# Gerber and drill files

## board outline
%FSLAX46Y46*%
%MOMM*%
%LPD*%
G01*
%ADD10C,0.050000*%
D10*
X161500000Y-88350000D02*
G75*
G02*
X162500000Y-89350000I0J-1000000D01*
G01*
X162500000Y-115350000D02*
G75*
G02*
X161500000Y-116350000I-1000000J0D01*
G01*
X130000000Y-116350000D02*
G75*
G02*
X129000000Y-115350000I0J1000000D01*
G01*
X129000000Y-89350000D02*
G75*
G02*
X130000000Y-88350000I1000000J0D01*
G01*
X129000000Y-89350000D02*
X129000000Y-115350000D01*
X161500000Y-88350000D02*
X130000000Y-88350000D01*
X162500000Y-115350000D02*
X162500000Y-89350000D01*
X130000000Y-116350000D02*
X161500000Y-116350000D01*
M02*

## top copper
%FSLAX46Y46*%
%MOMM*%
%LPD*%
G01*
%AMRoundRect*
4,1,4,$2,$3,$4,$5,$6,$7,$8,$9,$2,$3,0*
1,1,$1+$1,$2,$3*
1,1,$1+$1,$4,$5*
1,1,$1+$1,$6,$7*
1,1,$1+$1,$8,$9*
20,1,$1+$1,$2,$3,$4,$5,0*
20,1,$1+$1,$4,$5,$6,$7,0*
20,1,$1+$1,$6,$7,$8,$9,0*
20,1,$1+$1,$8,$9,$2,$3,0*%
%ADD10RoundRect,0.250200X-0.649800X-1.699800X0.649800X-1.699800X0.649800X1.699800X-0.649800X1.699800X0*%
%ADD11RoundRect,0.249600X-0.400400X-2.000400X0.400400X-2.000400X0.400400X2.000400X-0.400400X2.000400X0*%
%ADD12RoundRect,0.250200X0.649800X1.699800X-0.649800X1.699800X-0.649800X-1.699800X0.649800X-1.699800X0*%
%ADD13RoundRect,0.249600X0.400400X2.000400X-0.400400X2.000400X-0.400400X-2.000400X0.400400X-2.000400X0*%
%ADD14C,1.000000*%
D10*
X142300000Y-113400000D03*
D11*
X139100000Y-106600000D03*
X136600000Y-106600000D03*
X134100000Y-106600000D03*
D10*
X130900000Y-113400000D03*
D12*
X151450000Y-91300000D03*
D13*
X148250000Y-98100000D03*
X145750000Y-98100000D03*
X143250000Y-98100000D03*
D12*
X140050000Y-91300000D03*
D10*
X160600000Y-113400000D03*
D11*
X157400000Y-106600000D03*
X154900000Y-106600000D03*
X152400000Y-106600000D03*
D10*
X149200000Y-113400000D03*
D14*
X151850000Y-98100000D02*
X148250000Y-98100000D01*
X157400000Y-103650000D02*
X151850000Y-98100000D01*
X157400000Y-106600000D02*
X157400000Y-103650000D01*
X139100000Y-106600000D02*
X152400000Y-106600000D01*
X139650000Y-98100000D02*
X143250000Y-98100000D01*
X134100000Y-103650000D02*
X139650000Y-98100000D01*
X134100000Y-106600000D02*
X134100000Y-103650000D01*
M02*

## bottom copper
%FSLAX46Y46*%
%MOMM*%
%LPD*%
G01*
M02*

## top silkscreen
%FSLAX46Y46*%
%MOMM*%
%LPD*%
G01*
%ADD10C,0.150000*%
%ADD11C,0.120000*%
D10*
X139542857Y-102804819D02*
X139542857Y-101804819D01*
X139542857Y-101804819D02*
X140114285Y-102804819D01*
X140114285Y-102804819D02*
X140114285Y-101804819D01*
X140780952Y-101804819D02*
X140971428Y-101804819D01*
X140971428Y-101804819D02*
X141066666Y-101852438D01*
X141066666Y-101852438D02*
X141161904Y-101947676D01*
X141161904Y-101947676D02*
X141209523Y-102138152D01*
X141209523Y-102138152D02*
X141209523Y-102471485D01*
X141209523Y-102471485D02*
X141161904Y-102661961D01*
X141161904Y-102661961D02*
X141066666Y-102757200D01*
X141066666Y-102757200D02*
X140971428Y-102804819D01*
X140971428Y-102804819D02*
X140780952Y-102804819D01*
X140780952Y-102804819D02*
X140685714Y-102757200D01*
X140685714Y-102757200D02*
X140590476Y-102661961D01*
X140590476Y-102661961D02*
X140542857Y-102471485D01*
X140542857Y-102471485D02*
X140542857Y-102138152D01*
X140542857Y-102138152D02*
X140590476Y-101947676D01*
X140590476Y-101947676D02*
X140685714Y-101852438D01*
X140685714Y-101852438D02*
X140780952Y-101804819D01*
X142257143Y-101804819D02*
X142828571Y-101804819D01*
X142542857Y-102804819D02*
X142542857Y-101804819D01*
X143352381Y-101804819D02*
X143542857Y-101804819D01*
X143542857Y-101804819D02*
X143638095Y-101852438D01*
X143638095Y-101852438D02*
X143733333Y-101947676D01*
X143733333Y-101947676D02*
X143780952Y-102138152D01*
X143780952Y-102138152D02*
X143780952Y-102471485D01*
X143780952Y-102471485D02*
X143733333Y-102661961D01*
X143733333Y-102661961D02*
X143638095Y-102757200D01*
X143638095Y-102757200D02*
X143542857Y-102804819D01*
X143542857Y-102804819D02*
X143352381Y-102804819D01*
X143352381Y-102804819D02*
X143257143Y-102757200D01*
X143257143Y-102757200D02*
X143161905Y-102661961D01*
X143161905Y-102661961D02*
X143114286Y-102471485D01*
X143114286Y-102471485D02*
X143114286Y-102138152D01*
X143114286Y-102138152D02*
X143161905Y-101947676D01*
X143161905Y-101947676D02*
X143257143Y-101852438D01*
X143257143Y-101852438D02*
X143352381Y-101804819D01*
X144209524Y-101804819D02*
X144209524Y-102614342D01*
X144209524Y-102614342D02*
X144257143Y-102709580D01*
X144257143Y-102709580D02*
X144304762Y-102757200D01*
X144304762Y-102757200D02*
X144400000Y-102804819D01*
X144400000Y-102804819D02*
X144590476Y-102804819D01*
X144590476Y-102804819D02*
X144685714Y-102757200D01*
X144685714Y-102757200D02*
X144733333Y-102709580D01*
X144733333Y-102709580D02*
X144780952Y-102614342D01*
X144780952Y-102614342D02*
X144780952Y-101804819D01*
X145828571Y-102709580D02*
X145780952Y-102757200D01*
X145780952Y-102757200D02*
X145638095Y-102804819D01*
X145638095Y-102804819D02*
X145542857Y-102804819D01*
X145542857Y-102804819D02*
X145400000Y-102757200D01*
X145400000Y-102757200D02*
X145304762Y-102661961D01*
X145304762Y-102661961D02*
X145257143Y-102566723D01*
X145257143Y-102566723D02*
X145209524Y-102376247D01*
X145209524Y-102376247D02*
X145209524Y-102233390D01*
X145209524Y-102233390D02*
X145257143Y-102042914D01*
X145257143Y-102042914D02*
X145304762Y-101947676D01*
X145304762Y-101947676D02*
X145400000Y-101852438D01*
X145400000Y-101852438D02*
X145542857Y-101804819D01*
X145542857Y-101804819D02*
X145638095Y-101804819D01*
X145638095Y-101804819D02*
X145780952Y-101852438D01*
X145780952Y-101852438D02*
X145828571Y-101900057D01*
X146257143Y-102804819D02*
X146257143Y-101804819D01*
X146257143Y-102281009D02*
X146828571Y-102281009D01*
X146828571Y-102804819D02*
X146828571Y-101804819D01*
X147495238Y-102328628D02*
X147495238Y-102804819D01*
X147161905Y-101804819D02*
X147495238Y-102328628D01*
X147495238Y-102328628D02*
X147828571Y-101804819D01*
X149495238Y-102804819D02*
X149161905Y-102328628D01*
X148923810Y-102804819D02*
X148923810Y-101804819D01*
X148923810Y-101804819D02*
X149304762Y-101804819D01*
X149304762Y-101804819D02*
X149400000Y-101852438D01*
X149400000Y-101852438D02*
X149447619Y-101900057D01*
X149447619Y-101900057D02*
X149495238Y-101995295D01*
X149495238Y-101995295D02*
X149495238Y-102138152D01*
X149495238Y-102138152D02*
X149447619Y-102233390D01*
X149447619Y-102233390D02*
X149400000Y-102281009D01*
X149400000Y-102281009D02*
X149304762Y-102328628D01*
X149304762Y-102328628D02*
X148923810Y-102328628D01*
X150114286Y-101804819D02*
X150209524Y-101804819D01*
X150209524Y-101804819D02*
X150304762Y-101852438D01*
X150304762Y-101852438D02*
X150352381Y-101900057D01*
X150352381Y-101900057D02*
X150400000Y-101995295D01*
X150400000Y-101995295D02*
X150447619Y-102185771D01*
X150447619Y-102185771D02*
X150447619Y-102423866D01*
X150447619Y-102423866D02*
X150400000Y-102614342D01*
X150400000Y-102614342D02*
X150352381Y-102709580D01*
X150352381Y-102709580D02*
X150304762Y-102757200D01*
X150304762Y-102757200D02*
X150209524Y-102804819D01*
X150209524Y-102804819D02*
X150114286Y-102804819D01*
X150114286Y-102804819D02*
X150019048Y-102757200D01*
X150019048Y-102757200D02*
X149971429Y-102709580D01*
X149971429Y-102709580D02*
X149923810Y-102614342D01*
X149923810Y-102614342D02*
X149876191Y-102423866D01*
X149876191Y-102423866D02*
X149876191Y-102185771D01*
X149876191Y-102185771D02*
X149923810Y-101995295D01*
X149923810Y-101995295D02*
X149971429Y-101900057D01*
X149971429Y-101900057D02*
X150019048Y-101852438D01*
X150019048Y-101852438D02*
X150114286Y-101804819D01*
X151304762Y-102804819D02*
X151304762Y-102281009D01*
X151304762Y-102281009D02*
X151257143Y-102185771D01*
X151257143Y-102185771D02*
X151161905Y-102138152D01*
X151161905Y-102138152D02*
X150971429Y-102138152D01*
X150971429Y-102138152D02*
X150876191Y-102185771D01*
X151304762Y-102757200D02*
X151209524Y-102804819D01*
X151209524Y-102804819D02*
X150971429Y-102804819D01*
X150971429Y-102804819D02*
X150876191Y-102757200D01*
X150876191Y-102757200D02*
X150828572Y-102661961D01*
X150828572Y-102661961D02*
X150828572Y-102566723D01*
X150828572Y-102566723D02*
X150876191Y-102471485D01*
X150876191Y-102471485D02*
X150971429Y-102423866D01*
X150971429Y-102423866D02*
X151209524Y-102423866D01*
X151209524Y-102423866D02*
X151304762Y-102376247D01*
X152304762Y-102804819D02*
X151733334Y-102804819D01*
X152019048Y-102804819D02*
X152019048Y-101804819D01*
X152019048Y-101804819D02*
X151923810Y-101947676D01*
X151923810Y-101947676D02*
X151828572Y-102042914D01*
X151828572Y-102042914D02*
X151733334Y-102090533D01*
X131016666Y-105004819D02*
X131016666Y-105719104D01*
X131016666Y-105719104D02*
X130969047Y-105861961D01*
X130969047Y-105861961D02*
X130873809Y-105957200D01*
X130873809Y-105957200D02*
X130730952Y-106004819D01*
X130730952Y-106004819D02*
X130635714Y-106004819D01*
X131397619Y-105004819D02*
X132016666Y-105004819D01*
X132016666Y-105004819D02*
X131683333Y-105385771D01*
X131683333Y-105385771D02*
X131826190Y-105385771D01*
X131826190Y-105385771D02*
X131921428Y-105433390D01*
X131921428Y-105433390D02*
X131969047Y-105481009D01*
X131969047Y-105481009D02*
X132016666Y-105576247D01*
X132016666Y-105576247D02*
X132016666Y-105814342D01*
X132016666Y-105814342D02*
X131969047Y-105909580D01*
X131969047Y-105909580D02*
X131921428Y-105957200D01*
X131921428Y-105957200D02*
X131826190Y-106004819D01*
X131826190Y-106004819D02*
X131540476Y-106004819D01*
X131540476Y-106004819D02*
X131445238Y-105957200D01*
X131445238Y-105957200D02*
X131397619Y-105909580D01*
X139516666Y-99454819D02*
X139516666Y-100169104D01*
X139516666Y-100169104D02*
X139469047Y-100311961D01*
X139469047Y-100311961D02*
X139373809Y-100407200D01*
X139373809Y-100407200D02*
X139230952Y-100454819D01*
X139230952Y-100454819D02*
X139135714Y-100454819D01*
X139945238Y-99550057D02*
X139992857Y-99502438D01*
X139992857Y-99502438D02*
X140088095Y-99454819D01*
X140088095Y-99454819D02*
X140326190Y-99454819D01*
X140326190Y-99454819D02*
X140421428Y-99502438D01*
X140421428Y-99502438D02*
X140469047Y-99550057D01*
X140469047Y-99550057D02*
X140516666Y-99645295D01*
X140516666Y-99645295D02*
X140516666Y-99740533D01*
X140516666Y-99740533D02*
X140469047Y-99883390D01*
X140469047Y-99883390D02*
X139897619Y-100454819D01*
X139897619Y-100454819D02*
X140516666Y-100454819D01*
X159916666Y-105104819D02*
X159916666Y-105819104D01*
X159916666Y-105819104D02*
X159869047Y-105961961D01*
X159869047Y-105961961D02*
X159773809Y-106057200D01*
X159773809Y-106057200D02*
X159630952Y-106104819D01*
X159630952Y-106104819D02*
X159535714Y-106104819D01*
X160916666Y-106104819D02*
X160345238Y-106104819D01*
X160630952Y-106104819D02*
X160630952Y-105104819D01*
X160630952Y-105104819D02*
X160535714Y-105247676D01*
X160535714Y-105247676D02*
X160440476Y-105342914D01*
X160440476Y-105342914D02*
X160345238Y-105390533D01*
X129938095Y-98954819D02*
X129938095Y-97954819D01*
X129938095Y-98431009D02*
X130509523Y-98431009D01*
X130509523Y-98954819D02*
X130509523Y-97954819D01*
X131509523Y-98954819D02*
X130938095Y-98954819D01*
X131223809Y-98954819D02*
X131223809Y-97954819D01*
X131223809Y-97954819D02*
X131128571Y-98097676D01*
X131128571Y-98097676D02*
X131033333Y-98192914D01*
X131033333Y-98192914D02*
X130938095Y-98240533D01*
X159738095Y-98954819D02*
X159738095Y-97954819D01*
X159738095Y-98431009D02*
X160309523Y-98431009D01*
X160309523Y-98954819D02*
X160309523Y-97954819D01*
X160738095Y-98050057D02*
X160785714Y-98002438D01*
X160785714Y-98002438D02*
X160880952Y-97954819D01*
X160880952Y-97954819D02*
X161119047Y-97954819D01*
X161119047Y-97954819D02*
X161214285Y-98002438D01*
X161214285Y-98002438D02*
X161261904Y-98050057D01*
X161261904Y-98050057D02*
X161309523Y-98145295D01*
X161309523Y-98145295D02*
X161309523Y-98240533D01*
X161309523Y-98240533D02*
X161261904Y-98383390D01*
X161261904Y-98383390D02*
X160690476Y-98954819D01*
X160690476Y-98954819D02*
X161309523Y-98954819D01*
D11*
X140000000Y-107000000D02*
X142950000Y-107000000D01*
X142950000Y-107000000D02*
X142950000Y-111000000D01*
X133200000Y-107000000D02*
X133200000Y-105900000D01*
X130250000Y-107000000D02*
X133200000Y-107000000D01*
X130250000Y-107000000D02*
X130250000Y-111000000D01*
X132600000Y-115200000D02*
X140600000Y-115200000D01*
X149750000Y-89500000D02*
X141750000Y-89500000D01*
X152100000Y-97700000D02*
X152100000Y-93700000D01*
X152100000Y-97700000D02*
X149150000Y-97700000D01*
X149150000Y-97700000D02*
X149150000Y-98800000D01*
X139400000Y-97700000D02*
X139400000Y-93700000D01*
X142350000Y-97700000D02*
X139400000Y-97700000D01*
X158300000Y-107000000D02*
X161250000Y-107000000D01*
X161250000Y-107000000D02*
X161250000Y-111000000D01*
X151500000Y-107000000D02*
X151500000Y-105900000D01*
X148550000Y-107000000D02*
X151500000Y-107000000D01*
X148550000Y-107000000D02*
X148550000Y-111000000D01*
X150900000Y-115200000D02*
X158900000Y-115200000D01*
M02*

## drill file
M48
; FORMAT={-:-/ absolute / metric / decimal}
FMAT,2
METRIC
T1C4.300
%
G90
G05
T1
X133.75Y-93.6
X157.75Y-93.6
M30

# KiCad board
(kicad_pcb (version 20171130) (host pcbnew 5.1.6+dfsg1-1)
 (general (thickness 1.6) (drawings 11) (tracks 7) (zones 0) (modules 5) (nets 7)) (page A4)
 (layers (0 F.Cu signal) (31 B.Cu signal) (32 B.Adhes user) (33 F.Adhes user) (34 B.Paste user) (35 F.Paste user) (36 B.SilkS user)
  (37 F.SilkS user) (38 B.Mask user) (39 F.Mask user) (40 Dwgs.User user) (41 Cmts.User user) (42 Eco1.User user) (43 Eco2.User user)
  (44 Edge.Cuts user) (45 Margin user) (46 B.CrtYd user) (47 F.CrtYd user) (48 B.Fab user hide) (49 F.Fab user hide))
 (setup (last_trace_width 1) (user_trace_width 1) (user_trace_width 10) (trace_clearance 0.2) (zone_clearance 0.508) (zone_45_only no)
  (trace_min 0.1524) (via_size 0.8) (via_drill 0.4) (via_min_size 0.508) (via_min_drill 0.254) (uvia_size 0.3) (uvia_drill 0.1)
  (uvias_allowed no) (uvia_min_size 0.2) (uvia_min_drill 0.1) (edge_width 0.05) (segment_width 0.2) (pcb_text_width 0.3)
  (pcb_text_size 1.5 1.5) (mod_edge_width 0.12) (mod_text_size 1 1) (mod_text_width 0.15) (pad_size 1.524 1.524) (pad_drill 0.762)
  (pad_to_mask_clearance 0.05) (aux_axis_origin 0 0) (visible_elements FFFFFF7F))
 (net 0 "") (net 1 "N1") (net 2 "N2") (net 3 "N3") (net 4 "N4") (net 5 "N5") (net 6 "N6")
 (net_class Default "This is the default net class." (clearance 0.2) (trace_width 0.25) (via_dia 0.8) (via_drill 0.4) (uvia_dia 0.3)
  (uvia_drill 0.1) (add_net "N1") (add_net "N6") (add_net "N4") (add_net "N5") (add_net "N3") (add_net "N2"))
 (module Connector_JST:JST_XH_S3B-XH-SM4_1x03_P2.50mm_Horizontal (layer F.Cu) (at 136.6 111.1)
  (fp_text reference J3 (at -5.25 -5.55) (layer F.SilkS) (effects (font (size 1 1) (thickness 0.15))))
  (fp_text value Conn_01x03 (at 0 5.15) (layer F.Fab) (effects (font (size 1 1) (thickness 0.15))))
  (fp_line (start 3.4 -4.1) (end 6.35 -4.1) (layer F.SilkS) (width 0.12))
  (fp_line (start 6.35 -4.1) (end 6.35 -0.1) (layer F.SilkS) (width 0.12))
  (fp_line (start -3.4 -4.1) (end -3.4 -5.2) (layer F.SilkS) (width 0.12))
  (fp_line (start -6.35 -4.1) (end -3.4 -4.1) (layer F.SilkS) (width 0.12))
  (fp_line (start -6.35 -4.1) (end -6.35 -0.1) (layer F.SilkS) (width 0.12))
  (fp_line (start -4 4.1) (end 4 4.1) (layer F.SilkS) (width 0.12))
  (pad MP smd roundrect (at 5.7 2.3) (size 1.8 3.9) (layers F.Cu F.Paste F.Mask) (roundrect_rratio 0.139))
  (pad 3 smd roundrect (at 2.5 -4.5) (size 1.3 4.5) (layers F.Cu F.Paste F.Mask) (roundrect_rratio 0.192) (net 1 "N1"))
  (pad 2 smd roundrect (at 0 -4.5) (size 1.3 4.5) (layers F.Cu F.Paste F.Mask) (roundrect_rratio 0.192) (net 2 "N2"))
  (pad 1 smd roundrect (at -2.5 -4.5) (size 1.3 4.5) (layers F.Cu F.Paste F.Mask) (roundrect_rratio 0.192) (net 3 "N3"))
  (pad MP smd roundrect (at -5.7 2.3) (size 1.8 3.9) (layers F.Cu F.Paste F.Mask) (roundrect_rratio 0.139)))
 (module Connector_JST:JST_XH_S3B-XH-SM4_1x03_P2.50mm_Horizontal (layer F.Cu) (at 145.75 93.6 180)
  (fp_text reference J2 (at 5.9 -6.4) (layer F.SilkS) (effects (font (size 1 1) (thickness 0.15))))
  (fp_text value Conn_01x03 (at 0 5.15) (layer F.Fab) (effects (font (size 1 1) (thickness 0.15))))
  (fp_line (start -4 4.1) (end 4 4.1) (layer F.SilkS) (width 0.12))
  (fp_line (start -6.35 -4.1) (end -6.35 -0.1) (layer F.SilkS) (width 0.12))
  (fp_line (start -6.35 -4.1) (end -3.4 -4.1) (layer F.SilkS) (width 0.12))
  (fp_line (start -3.4 -4.1) (end -3.4 -5.2) (layer F.SilkS) (width 0.12))
  (fp_line (start 6.35 -4.1) (end 6.35 -0.1) (layer F.SilkS) (width 0.12))
  (fp_line (start 3.4 -4.1) (end 6.35 -4.1) (layer F.SilkS) (width 0.12))
  (pad MP smd roundrect (at -5.7 2.3 180) (size 1.8 3.9) (layers F.Cu F.Paste F.Mask) (roundrect_rratio 0.139))
  (pad 1 smd roundrect (at -2.5 -4.5 180) (size 1.3 4.5) (layers F.Cu F.Paste F.Mask) (roundrect_rratio 0.192) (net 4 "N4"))
  (pad 2 smd roundrect (at 0 -4.5 180) (size 1.3 4.5) (layers F.Cu F.Paste F.Mask) (roundrect_rratio 0.192) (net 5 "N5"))
  (pad 3 smd roundrect (at 2.5 -4.5 180) (size 1.3 4.5) (layers F.Cu F.Paste F.Mask) (roundrect_rratio 0.192) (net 3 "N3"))
  (pad MP smd roundrect (at 5.7 2.3 180) (size 1.8 3.9) (layers F.Cu F.Paste F.Mask) (roundrect_rratio 0.139)))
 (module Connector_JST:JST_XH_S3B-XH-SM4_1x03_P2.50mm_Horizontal (layer F.Cu) (at 154.9 111.1)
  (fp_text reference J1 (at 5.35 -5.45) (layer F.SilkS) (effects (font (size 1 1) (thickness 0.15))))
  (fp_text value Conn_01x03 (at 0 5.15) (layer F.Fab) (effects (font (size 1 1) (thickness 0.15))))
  (fp_line (start 3.4 -4.1) (end 6.35 -4.1) (layer F.SilkS) (width 0.12))
  (fp_line (start 6.35 -4.1) (end 6.35 -0.1) (layer F.SilkS) (width 0.12))
  (fp_line (start -3.4 -4.1) (end -3.4 -5.2) (layer F.SilkS) (width 0.12))
  (fp_line (start -6.35 -4.1) (end -3.4 -4.1) (layer F.SilkS) (width 0.12))
  (fp_line (start -6.35 -4.1) (end -6.35 -0.1) (layer F.SilkS) (width 0.12))
  (fp_line (start -4 4.1) (end 4 4.1) (layer F.SilkS) (width 0.12))
  (pad MP smd roundrect (at 5.7 2.3) (size 1.8 3.9) (layers F.Cu F.Paste F.Mask) (roundrect_rratio 0.139))
  (pad 3 smd roundrect (at 2.5 -4.5) (size 1.3 4.5) (layers F.Cu F.Paste F.Mask) (roundrect_rratio 0.192) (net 4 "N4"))
  (pad 2 smd roundrect (at 0 -4.5) (size 1.3 4.5) (layers F.Cu F.Paste F.Mask) (roundrect_rratio 0.192) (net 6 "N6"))
  (pad 1 smd roundrect (at -2.5 -4.5) (size 1.3 4.5) (layers F.Cu F.Paste F.Mask) (roundrect_rratio 0.192) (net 1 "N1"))
  (pad MP smd roundrect (at -5.7 2.3) (size 1.8 3.9) (layers F.Cu F.Paste F.Mask) (roundrect_rratio 0.139)))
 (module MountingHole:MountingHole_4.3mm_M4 (layer F.Cu) (at 133.75 93.6)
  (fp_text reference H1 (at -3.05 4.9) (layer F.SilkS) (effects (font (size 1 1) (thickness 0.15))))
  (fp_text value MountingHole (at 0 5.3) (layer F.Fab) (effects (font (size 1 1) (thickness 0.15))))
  (pad 1 np_thru_hole circle (at 0 0) (size 4.3 4.3) (drill 4.3) (layers *.Cu *.Mask)))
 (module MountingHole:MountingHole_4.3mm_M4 (layer F.Cu) (at 157.75 93.6)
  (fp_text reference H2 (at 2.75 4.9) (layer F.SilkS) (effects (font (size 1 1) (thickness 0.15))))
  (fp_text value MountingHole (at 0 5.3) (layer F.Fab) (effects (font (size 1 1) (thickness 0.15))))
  (pad 1 np_thru_hole circle (at 0 0) (size 4.3 4.3) (drill 4.3) (layers *.Cu *.Mask)))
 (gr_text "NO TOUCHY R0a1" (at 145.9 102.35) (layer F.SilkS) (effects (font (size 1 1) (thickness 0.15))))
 (gr_arc (start 161.5 89.35) (end 162.5 89.35) (angle -90) (layer Edge.Cuts) (width 0.05))
 (gr_arc (start 161.5 115.35) (end 161.5 116.35) (angle -90) (layer Edge.Cuts) (width 0.05))
 (gr_arc (start 130 115.35) (end 129 115.35) (angle -90) (layer Edge.Cuts) (width 0.05))
 (gr_arc (start 130 89.35) (end 130 88.35) (angle -90) (layer Edge.Cuts) (width 0.05))
 (gr_line (start 129 89.35) (end 129 115.35) (layer Edge.Cuts) (width 0.05))
 (gr_line (start 161.5 88.35) (end 130 88.35) (layer Edge.Cuts) (width 0.05))
 (gr_line (start 162.5 115.35) (end 162.5 89.35) (layer Edge.Cuts) (width 0.05))
 (gr_line (start 130 116.35) (end 161.5 116.35) (layer Edge.Cuts) (width 0.05))
 (segment (start 151.85 98.1) (end 148.25 98.1) (width 1) (layer F.Cu) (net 4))
 (segment (start 157.4 103.65) (end 151.85 98.1) (width 1) (layer F.Cu) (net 4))
 (segment (start 157.4 106.6) (end 157.4 103.65) (width 1) (layer F.Cu) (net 4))
 (segment (start 139.1 106.6) (end 152.4 106.6) (width 1) (layer F.Cu) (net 1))
 (segment (start 139.65 98.1) (end 143.25 98.1) (width 1) (layer F.Cu) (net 3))
 (segment (start 134.1 103.65) (end 139.65 98.1) (width 1) (layer F.Cu) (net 3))
 (segment (start 134.1 106.6) (end 134.1 103.65) (width 1) (layer F.Cu) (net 3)))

